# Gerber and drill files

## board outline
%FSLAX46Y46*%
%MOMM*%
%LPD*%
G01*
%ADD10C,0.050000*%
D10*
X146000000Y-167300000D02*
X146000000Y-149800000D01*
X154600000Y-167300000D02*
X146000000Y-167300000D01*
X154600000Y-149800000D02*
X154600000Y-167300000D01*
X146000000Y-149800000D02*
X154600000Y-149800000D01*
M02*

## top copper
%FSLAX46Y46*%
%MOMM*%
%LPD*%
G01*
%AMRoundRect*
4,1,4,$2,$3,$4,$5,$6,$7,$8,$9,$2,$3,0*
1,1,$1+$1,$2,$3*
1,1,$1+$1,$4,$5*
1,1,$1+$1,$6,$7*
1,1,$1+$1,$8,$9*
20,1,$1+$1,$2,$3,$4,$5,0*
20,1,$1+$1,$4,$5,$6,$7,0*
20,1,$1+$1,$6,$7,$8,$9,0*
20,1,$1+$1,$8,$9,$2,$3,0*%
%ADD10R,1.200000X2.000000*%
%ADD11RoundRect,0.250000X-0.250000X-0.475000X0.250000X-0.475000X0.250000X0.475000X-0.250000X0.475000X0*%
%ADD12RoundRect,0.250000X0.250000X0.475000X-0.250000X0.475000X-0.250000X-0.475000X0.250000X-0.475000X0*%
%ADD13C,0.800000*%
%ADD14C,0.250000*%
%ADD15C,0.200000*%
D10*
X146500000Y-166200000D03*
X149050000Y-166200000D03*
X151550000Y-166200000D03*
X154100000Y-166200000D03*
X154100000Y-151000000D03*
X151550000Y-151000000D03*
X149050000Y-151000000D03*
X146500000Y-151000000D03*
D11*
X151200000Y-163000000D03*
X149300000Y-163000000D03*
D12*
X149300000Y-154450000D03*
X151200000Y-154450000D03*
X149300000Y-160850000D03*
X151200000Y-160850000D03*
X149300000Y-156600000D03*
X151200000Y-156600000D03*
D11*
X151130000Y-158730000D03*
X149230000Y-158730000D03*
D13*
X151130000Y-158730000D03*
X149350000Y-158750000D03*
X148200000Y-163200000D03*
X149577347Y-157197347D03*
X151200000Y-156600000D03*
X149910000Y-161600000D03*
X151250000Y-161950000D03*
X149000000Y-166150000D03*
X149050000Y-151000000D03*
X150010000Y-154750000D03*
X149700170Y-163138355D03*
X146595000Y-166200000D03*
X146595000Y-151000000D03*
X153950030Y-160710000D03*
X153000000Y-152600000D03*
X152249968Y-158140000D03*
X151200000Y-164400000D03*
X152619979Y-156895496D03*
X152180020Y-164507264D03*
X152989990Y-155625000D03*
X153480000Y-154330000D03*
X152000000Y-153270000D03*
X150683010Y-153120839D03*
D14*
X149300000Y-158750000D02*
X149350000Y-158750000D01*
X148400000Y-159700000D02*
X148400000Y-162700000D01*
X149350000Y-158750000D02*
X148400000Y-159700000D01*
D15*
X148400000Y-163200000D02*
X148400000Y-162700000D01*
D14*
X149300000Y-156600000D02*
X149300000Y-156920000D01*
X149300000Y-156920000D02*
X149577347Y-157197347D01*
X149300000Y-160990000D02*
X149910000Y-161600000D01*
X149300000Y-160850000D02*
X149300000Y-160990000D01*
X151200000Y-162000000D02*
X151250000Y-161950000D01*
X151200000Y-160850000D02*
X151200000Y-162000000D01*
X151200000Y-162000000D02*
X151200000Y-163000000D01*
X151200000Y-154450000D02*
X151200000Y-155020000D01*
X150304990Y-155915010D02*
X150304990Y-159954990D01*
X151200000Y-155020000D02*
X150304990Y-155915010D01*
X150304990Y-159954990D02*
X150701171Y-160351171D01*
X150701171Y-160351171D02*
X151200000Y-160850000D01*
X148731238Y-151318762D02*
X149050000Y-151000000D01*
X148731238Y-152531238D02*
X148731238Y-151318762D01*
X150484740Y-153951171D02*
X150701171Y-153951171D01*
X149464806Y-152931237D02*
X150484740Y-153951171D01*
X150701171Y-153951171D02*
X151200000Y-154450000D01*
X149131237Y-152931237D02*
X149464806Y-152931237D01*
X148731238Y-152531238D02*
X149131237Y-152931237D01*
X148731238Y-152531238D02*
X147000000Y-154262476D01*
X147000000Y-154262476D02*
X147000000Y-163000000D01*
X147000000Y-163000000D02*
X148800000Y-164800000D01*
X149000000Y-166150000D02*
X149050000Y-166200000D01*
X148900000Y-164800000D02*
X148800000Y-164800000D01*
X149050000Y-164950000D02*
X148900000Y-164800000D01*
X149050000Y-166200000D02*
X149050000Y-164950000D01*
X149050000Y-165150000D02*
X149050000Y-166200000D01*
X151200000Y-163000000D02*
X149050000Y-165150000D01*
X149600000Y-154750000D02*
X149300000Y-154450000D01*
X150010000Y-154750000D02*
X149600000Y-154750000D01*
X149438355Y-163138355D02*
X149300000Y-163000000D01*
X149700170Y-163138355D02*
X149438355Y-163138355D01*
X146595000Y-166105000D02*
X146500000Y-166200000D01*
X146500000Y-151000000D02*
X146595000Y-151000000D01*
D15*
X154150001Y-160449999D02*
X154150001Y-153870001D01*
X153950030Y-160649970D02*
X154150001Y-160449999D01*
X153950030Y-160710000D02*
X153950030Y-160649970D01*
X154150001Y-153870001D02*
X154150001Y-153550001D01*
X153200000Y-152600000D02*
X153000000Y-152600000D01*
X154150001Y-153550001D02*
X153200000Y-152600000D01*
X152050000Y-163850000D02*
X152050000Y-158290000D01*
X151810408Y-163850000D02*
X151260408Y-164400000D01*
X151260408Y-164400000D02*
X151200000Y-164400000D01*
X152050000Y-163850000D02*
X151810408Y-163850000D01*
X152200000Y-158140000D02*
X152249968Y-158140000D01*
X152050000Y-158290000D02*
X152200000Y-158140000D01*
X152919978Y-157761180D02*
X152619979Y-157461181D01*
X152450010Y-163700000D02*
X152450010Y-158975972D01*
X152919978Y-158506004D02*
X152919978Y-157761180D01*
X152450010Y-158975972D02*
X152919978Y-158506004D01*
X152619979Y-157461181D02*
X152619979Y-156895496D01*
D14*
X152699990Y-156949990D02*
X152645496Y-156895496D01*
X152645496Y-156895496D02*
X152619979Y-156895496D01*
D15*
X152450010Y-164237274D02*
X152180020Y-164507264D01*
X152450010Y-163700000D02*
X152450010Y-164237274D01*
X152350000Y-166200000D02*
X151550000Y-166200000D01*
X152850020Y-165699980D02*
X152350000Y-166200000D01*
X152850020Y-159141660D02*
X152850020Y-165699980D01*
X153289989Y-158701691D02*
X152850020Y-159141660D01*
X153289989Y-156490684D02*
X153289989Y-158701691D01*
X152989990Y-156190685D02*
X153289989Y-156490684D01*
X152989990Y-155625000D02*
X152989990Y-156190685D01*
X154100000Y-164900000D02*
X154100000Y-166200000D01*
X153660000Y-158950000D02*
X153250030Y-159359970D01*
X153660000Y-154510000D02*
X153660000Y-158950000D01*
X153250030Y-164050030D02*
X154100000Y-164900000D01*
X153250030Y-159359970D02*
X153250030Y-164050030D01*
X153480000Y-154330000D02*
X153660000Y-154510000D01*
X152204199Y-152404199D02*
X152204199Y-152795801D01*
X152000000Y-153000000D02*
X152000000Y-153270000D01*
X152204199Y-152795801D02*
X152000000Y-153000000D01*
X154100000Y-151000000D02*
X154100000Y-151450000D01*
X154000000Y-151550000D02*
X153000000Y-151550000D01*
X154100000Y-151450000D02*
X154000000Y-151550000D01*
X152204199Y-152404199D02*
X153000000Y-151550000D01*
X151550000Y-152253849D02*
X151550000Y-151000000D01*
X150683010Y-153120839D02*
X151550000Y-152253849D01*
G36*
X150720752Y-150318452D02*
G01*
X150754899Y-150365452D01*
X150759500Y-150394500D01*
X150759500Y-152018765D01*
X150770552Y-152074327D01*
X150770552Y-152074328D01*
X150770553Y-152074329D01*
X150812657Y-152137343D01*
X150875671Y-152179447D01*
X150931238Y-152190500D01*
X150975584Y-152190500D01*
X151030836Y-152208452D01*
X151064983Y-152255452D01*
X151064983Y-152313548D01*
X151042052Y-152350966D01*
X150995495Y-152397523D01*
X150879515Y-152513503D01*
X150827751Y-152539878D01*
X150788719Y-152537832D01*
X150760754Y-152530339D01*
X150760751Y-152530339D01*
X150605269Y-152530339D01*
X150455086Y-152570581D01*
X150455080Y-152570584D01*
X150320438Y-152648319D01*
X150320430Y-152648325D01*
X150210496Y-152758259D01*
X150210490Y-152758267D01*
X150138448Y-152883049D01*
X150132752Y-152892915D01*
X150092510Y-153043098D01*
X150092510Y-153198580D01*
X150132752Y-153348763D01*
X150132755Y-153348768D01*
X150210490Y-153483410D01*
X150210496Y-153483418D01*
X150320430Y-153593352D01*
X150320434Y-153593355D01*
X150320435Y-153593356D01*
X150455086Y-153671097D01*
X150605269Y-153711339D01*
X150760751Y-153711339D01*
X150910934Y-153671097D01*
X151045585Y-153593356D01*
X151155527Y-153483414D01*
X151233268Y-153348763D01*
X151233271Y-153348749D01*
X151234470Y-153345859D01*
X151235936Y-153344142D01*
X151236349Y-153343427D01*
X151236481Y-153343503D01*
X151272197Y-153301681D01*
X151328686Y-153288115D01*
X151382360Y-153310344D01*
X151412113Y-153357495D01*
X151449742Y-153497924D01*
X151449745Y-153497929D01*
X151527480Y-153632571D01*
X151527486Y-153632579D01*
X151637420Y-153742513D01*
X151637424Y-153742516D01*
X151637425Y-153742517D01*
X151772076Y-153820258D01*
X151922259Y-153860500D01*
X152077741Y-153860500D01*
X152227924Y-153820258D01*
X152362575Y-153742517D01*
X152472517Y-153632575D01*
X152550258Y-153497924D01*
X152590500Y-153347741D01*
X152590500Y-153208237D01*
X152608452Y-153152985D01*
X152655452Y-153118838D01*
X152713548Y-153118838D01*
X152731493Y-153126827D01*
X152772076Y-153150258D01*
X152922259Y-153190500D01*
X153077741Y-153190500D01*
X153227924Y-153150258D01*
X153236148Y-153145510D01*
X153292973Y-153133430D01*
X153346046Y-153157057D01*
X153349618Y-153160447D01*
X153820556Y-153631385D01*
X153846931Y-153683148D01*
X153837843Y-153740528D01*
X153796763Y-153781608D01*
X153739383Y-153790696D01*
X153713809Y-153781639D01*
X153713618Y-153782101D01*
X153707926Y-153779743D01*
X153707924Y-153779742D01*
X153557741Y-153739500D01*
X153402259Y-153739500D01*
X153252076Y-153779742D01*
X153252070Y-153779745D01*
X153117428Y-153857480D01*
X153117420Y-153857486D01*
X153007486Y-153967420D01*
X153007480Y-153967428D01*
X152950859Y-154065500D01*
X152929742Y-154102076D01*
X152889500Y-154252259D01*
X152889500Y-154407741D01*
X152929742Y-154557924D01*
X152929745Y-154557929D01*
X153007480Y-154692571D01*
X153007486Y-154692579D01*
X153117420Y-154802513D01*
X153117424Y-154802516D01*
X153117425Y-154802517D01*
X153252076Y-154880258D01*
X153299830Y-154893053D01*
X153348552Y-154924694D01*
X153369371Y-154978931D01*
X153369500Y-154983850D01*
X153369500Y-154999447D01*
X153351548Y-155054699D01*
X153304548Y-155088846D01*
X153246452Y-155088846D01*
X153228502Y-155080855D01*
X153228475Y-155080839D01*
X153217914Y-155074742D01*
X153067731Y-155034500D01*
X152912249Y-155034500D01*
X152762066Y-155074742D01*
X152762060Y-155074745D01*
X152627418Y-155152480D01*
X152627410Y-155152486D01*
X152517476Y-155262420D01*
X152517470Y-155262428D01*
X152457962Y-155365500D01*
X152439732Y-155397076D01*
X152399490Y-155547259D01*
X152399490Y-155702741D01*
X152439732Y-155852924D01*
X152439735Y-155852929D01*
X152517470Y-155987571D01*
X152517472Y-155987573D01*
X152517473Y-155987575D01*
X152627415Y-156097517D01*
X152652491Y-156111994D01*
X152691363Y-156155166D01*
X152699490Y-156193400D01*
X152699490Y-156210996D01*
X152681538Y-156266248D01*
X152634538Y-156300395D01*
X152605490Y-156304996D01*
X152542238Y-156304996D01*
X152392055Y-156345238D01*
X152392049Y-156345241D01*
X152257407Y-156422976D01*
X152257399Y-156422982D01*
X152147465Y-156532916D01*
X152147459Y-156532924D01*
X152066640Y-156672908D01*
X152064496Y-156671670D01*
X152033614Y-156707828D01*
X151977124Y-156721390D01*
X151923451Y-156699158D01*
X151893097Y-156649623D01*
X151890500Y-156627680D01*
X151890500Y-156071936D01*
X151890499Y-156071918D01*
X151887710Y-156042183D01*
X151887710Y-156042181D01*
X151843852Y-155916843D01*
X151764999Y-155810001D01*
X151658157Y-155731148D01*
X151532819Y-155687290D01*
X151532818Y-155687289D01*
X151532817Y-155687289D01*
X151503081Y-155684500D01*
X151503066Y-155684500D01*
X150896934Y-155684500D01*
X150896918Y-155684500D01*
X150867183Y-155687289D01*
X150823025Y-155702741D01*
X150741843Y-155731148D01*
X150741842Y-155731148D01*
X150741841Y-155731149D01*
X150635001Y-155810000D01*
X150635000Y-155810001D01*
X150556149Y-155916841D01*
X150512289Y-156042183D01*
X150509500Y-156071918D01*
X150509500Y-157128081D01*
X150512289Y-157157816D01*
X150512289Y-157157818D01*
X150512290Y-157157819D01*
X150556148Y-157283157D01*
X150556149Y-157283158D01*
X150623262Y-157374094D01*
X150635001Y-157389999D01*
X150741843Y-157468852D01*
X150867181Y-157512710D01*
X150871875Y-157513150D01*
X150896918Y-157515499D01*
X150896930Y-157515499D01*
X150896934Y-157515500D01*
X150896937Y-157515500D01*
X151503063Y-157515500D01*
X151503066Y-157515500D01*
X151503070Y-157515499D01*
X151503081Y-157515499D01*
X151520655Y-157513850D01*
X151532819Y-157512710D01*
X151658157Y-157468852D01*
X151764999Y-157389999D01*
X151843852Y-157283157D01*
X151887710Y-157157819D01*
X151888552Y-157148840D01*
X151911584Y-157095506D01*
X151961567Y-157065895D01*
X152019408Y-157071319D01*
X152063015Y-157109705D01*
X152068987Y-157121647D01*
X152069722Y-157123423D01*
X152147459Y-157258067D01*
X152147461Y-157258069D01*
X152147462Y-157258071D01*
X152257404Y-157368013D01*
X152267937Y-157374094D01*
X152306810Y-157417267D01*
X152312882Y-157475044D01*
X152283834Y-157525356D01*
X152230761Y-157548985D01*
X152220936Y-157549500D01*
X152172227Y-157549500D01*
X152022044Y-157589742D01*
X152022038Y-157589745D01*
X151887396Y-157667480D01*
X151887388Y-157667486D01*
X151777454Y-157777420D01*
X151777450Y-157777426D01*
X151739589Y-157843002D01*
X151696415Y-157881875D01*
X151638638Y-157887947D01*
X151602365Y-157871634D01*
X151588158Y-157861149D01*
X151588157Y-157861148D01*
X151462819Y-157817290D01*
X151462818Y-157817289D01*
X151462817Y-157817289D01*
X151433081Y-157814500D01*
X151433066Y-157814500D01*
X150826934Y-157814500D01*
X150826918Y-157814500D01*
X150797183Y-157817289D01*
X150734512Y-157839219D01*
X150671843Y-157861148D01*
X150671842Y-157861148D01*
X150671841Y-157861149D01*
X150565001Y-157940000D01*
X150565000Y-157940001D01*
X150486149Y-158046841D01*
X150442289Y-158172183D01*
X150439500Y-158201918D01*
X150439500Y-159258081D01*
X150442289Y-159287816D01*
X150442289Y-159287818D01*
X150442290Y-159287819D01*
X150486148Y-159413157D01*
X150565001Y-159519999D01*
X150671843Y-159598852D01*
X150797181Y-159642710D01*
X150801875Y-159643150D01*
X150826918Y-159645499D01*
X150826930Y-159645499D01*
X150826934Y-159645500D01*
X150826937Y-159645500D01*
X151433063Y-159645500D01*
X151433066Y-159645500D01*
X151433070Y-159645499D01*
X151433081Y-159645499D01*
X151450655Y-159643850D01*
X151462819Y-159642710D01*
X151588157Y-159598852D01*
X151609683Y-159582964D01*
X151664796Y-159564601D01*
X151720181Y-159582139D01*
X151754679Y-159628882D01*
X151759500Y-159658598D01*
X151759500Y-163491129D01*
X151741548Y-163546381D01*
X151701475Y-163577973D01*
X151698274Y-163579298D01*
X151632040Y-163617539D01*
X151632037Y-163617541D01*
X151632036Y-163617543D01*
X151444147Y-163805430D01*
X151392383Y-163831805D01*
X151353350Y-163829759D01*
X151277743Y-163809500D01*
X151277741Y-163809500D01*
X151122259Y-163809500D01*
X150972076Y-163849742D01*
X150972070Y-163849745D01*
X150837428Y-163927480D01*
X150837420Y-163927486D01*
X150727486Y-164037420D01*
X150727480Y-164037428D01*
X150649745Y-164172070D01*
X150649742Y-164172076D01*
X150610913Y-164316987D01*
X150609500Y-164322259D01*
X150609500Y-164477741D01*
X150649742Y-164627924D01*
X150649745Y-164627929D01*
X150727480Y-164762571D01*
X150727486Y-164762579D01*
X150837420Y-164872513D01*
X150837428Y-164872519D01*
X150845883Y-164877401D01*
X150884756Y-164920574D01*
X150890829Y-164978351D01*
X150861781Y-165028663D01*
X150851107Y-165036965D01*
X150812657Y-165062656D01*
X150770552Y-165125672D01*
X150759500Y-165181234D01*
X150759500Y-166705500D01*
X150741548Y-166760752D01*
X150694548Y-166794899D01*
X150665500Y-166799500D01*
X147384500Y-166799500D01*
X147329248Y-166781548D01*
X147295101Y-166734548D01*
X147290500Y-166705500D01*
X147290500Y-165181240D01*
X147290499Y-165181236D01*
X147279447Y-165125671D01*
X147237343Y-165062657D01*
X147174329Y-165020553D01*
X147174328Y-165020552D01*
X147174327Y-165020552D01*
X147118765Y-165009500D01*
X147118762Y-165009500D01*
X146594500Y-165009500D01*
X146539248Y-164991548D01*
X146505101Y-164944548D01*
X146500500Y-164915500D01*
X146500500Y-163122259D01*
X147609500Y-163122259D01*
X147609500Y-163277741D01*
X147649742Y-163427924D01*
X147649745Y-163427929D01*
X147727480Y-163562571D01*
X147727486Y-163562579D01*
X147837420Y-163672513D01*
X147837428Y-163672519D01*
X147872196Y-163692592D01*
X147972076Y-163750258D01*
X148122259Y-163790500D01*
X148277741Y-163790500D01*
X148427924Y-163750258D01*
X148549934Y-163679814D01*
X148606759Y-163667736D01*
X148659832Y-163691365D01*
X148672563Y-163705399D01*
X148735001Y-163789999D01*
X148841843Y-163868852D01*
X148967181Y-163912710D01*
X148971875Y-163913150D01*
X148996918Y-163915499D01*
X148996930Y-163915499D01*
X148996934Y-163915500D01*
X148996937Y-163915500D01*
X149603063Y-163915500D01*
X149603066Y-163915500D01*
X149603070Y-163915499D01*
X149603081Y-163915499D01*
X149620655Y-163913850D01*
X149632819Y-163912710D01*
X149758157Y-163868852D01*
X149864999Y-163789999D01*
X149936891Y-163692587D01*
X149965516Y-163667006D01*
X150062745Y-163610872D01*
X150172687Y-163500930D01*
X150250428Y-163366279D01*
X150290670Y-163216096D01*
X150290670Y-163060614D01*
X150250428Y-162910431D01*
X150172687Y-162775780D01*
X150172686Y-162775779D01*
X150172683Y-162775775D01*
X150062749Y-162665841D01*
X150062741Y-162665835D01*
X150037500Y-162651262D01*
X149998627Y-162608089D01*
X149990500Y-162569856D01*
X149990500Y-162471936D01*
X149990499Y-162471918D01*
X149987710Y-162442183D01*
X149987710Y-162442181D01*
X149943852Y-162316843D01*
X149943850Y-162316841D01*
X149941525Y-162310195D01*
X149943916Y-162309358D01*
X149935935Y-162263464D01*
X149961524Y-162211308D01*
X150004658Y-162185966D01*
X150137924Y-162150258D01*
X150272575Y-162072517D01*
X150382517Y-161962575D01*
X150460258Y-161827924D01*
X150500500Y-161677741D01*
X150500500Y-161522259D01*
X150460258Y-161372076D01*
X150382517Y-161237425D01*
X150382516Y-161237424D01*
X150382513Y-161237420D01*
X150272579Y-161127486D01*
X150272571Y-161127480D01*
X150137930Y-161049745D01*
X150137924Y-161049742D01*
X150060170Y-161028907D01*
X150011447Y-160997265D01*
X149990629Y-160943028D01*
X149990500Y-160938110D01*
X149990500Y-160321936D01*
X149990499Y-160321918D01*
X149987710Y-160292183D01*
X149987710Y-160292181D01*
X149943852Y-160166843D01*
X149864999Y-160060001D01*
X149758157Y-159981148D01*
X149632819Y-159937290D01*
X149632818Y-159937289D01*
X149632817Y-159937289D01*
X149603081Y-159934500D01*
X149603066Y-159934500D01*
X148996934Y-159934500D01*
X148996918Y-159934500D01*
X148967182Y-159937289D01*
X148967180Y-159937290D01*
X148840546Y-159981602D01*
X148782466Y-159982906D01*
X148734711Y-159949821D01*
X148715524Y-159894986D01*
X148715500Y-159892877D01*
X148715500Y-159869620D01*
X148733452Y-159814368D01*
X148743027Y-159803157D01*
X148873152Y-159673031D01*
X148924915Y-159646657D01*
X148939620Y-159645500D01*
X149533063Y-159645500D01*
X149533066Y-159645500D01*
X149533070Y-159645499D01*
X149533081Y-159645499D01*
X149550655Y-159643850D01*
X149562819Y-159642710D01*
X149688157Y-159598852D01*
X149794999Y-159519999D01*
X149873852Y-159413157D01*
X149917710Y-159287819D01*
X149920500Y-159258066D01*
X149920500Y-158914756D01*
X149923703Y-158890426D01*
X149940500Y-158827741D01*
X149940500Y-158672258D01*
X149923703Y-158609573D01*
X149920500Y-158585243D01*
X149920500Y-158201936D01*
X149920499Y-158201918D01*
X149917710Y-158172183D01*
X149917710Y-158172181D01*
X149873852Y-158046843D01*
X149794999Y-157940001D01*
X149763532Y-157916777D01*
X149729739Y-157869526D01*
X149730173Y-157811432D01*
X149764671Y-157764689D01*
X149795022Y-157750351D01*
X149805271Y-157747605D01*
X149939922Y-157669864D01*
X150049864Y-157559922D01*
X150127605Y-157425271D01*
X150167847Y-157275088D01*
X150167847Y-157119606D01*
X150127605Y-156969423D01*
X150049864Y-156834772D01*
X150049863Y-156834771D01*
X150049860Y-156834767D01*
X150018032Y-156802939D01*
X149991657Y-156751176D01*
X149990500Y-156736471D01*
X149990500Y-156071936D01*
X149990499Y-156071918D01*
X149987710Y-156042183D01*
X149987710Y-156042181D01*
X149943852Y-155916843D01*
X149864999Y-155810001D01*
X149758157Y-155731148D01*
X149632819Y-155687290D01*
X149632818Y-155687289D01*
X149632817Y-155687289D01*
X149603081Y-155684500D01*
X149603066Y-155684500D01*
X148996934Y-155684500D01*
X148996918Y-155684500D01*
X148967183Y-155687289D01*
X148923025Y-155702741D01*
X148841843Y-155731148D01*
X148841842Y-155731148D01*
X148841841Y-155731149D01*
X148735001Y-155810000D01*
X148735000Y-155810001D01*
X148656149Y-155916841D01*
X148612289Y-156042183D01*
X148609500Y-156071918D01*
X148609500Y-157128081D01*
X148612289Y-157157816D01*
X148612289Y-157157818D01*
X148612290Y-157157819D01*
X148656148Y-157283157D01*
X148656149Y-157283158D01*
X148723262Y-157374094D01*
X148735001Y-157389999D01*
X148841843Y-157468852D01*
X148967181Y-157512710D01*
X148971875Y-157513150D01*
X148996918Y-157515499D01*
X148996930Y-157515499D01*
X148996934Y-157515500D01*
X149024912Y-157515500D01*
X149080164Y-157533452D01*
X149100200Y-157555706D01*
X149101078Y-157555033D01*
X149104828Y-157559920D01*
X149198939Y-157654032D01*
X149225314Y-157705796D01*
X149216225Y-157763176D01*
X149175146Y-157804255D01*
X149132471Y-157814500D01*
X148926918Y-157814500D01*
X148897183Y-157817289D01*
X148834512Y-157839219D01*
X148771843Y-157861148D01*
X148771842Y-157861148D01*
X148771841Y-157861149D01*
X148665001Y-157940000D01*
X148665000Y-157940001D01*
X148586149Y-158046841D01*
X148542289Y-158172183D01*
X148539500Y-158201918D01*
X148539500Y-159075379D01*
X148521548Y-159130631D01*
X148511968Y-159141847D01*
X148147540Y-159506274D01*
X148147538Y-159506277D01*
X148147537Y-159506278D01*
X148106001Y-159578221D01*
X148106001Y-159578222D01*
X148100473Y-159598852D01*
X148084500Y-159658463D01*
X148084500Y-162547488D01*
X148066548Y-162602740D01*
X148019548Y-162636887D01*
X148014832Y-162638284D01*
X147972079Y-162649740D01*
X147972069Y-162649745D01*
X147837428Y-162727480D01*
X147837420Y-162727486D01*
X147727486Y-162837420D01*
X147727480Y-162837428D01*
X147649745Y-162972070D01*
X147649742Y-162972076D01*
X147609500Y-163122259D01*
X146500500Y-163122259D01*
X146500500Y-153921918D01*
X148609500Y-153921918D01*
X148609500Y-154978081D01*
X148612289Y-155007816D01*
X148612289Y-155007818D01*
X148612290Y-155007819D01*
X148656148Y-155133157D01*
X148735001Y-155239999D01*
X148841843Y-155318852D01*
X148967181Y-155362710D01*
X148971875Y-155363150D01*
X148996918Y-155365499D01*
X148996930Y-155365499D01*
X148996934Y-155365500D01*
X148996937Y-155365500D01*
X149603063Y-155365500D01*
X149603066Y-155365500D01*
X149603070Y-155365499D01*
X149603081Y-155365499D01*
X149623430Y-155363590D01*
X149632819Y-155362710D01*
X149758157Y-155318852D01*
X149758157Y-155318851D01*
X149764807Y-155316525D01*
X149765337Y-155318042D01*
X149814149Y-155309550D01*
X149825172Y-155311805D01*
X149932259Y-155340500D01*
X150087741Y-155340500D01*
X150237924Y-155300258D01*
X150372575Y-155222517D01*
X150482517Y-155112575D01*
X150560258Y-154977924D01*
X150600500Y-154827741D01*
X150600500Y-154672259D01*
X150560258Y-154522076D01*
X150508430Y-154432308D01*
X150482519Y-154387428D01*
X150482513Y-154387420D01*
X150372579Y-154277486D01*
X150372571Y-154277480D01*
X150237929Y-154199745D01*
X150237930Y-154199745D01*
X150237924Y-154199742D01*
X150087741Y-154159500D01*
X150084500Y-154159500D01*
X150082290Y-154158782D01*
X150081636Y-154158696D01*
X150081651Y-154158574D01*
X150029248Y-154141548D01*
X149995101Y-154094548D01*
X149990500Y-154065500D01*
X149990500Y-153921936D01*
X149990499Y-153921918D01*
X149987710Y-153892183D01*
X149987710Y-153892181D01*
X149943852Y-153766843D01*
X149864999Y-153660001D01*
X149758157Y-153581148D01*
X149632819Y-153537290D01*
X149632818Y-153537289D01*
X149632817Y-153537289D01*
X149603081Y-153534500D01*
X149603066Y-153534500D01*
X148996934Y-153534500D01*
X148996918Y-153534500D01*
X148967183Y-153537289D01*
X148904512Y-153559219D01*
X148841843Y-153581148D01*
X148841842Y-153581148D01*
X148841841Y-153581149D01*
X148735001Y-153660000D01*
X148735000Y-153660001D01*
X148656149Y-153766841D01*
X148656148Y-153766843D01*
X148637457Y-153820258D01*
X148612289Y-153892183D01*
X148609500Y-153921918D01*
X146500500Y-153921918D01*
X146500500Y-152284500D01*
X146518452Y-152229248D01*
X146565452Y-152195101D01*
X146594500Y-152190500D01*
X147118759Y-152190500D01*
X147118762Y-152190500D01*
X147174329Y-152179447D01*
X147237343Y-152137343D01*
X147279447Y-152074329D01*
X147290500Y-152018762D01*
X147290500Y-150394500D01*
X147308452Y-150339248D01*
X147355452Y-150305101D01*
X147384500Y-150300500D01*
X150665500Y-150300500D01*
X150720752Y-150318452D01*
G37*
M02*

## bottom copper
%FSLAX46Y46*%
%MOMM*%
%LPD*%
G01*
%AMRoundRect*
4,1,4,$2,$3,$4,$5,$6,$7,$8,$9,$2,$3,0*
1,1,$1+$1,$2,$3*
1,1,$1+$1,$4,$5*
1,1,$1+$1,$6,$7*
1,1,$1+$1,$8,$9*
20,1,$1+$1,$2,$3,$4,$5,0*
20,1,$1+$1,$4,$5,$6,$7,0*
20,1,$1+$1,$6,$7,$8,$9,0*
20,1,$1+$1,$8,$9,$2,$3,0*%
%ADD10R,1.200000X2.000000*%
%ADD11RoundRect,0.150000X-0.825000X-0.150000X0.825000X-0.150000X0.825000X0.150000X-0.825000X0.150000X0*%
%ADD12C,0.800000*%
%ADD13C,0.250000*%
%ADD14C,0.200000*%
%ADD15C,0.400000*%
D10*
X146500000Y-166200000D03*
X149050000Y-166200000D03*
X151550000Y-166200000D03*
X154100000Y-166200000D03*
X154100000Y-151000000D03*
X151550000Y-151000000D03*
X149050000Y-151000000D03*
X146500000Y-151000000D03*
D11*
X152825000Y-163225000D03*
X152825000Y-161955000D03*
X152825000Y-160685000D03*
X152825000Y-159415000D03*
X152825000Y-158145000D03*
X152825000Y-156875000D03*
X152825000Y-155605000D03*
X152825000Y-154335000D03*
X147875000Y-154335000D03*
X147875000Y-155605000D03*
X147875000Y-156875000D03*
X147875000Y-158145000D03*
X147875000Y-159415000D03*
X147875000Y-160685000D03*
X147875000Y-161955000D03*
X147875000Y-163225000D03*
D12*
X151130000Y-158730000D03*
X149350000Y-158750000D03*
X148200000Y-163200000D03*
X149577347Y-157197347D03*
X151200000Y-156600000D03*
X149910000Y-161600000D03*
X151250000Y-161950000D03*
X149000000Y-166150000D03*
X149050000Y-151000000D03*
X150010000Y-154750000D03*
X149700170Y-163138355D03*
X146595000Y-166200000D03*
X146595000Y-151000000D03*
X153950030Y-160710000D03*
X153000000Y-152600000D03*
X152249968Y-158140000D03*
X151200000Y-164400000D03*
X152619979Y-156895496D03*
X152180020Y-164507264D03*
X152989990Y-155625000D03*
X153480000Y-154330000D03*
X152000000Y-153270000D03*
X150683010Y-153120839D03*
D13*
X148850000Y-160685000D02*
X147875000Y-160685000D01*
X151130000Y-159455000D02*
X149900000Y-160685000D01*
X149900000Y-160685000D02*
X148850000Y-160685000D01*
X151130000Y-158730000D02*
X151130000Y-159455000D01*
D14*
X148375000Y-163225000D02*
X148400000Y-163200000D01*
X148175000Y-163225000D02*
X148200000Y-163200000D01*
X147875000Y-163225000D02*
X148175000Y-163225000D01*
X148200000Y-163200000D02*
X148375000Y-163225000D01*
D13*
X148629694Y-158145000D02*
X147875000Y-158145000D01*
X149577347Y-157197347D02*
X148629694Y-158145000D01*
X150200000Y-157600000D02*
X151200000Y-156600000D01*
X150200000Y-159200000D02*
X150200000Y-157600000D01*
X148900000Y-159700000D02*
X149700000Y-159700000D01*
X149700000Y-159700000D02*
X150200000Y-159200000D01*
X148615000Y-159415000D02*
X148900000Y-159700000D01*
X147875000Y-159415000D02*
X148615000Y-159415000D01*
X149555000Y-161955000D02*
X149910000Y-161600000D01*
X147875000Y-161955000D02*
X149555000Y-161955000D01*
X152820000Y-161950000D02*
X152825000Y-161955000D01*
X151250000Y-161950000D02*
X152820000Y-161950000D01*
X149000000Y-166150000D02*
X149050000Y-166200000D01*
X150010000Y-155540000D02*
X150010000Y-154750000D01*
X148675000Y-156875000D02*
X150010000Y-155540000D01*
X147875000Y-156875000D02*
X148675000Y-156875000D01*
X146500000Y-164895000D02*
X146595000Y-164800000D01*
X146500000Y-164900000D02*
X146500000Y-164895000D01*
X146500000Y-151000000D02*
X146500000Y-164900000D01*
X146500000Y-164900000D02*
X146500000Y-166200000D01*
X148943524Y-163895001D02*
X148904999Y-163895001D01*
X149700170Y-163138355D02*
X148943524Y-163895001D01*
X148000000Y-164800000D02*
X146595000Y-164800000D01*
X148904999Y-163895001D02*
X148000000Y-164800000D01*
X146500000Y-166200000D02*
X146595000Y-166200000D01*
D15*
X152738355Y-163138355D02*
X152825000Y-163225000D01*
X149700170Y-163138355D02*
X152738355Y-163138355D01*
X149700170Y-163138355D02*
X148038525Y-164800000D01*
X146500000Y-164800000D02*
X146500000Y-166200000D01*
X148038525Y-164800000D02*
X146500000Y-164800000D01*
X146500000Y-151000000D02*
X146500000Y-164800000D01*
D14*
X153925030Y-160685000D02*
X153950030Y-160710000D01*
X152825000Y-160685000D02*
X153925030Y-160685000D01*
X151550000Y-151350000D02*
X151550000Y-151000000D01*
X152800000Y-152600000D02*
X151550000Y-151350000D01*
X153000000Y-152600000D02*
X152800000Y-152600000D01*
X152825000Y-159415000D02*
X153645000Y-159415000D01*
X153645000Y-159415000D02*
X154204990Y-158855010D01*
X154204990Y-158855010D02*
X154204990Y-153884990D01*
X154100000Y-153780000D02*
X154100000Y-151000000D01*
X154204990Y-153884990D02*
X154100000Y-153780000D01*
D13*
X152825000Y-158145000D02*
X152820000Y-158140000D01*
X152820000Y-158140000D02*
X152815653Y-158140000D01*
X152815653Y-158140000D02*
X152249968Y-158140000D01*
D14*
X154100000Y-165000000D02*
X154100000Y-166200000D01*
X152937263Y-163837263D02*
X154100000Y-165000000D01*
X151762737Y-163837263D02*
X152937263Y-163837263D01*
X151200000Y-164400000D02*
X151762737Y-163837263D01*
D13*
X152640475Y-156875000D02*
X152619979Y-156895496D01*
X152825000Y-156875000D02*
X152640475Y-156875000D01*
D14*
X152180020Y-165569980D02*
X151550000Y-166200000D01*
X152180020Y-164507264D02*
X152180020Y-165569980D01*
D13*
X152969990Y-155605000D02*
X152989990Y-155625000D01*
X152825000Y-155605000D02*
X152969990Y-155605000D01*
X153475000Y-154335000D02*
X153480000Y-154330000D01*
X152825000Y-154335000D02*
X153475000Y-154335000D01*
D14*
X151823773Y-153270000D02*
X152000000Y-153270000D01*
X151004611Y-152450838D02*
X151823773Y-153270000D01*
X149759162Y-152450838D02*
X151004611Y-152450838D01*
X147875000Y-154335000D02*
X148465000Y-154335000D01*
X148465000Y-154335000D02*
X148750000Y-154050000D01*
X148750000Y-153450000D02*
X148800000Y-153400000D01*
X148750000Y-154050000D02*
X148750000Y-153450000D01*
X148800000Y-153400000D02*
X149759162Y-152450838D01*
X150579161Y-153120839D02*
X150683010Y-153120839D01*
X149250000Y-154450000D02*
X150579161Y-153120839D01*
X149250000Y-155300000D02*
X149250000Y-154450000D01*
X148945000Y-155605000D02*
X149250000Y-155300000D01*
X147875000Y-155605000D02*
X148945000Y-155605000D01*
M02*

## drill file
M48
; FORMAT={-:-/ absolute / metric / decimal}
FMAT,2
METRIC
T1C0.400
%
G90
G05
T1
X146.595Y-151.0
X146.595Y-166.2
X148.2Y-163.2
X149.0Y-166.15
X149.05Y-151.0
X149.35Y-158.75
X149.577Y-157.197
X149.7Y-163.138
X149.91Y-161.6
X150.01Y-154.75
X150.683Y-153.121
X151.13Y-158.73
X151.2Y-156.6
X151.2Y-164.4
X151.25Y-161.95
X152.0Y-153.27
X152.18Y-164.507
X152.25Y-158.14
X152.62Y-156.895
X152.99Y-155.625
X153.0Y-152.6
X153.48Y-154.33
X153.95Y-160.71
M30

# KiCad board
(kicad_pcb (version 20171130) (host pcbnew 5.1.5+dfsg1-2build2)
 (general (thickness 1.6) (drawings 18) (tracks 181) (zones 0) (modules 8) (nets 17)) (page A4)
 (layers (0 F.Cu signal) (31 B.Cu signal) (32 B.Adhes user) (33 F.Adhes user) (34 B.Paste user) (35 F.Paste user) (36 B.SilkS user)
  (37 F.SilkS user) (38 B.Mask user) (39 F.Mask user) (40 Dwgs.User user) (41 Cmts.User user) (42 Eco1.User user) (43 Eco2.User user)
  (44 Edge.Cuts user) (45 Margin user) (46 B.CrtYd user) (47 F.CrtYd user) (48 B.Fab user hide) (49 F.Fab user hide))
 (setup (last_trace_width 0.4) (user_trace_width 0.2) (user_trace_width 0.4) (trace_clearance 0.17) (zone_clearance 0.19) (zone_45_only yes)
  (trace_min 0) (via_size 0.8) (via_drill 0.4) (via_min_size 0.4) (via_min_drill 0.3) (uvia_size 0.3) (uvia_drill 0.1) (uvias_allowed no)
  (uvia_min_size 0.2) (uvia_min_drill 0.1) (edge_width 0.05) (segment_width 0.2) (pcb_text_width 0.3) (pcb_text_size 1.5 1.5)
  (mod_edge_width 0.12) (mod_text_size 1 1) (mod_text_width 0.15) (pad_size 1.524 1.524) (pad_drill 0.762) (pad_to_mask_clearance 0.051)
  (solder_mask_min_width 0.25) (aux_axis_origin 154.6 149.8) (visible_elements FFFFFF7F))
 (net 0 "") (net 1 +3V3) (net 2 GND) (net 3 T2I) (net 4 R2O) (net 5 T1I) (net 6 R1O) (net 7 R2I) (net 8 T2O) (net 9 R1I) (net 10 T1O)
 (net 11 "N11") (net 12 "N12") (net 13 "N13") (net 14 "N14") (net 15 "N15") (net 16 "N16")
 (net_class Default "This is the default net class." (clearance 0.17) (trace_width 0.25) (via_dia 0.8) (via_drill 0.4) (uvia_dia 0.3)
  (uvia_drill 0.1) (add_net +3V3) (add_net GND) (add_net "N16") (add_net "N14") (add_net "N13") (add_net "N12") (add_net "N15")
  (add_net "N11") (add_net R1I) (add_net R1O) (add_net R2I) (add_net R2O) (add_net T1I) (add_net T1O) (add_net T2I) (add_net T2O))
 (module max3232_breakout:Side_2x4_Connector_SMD (layer B.Cu) (at 150.3 166.2 270)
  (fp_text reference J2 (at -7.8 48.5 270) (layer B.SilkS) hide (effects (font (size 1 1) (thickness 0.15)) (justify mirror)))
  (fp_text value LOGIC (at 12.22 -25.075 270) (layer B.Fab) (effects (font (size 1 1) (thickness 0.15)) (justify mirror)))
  (pad 8 smd rect (at 0 3.8 270) (size 2 1.2) (layers F.Cu F.Paste F.Mask) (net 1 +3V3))
  (pad 6 smd rect (at 0 1.25 270) (size 2 1.2) (layers F.Cu F.Paste F.Mask) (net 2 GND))
  (pad 4 smd rect (at 0 -1.25 270) (size 2 1.2) (layers F.Cu F.Paste F.Mask) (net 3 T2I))
  (pad 2 smd rect (at 0 -3.8 270) (size 2 1.2) (layers F.Cu F.Paste F.Mask) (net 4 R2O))
  (pad 7 smd rect (at 0 3.8 270) (size 2 1.2) (layers B.Cu B.Paste B.Mask) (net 1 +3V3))
  (pad 5 smd rect (at 0 1.25 270) (size 2 1.2) (layers B.Cu B.Paste B.Mask) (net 2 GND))
  (pad 3 smd rect (at 0 -1.25 270) (size 2 1.2) (layers B.Cu B.Paste B.Mask) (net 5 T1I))
  (pad 1 smd rect (at 0 -3.8 270) (size 2 1.2) (layers B.Cu B.Paste B.Mask) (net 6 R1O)))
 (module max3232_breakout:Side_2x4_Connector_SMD (layer B.Cu) (at 150.3 151 90)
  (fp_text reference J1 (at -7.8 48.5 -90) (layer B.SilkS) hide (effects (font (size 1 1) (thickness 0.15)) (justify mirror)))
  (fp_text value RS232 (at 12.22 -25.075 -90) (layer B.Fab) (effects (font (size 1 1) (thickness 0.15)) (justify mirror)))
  (pad 8 smd rect (at 0 3.8 90) (size 2 1.2) (layers F.Cu F.Paste F.Mask) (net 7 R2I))
  (pad 6 smd rect (at 0 1.25 90) (size 2 1.2) (layers F.Cu F.Paste F.Mask) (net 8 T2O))
  (pad 4 smd rect (at 0 -1.25 90) (size 2 1.2) (layers F.Cu F.Paste F.Mask) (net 2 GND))
  (pad 2 smd rect (at 0 -3.8 90) (size 2 1.2) (layers F.Cu F.Paste F.Mask) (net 1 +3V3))
  (pad 7 smd rect (at 0 3.8 90) (size 2 1.2) (layers B.Cu B.Paste B.Mask) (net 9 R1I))
  (pad 5 smd rect (at 0 1.25 90) (size 2 1.2) (layers B.Cu B.Paste B.Mask) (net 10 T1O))
  (pad 3 smd rect (at 0 -1.25 90) (size 2 1.2) (layers B.Cu B.Paste B.Mask) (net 2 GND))
  (pad 1 smd rect (at 0 -3.8 90) (size 2 1.2) (layers B.Cu B.Paste B.Mask) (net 1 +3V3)))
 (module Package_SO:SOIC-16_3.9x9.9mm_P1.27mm (layer B.Cu) (at 150.35 158.78)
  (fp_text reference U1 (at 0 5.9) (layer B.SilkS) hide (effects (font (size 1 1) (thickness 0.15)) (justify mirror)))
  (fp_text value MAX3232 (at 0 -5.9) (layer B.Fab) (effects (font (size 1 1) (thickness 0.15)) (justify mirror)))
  (pad 16 smd roundrect (at 2.475 4.445) (size 1.95 0.6) (layers B.Cu B.Paste B.Mask) (roundrect_rratio 0.25) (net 1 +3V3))
  (pad 15 smd roundrect (at 2.475 3.175) (size 1.95 0.6) (layers B.Cu B.Paste B.Mask) (roundrect_rratio 0.25) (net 2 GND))
  (pad 14 smd roundrect (at 2.475 1.905) (size 1.95 0.6) (layers B.Cu B.Paste B.Mask) (roundrect_rratio 0.25) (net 10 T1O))
  (pad 13 smd roundrect (at 2.475 0.635) (size 1.95 0.6) (layers B.Cu B.Paste B.Mask) (roundrect_rratio 0.25) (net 9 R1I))
  (pad 12 smd roundrect (at 2.475 -0.635) (size 1.95 0.6) (layers B.Cu B.Paste B.Mask) (roundrect_rratio 0.25) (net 6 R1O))
  (pad 11 smd roundrect (at 2.475 -1.905) (size 1.95 0.6) (layers B.Cu B.Paste B.Mask) (roundrect_rratio 0.25) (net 5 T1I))
  (pad 10 smd roundrect (at 2.475 -3.175) (size 1.95 0.6) (layers B.Cu B.Paste B.Mask) (roundrect_rratio 0.25) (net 3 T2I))
  (pad 9 smd roundrect (at 2.475 -4.445) (size 1.95 0.6) (layers B.Cu B.Paste B.Mask) (roundrect_rratio 0.25) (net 4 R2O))
  (pad 8 smd roundrect (at -2.475 -4.445) (size 1.95 0.6) (layers B.Cu B.Paste B.Mask) (roundrect_rratio 0.25) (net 7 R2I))
  (pad 7 smd roundrect (at -2.475 -3.175) (size 1.95 0.6) (layers B.Cu B.Paste B.Mask) (roundrect_rratio 0.25) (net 8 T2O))
  (pad 6 smd roundrect (at -2.475 -1.905) (size 1.95 0.6) (layers B.Cu B.Paste B.Mask) (roundrect_rratio 0.25) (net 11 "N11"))
  (pad 5 smd roundrect (at -2.475 -0.635) (size 1.95 0.6) (layers B.Cu B.Paste B.Mask) (roundrect_rratio 0.25) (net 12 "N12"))
  (pad 4 smd roundrect (at -2.475 0.635) (size 1.95 0.6) (layers B.Cu B.Paste B.Mask) (roundrect_rratio 0.25) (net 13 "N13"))
  (pad 3 smd roundrect (at -2.475 1.905) (size 1.95 0.6) (layers B.Cu B.Paste B.Mask) (roundrect_rratio 0.25) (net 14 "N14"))
  (pad 2 smd roundrect (at -2.475 3.175) (size 1.95 0.6) (layers B.Cu B.Paste B.Mask) (roundrect_rratio 0.25) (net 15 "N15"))
  (pad 1 smd roundrect (at -2.475 4.445) (size 1.95 0.6) (layers B.Cu B.Paste B.Mask) (roundrect_rratio 0.25) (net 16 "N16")))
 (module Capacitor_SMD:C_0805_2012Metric (layer F.Cu) (at 150.25 163)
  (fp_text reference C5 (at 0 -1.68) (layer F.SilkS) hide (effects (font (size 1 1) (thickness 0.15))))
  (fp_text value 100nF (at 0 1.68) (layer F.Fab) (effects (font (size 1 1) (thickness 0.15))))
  (pad 2 smd roundrect (at 0.95 0) (size 1 1.45) (layers F.Cu F.Paste F.Mask) (roundrect_rratio 0.25) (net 2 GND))
  (pad 1 smd roundrect (at -0.95 0) (size 1 1.45) (layers F.Cu F.Paste F.Mask) (roundrect_rratio 0.25) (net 1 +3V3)))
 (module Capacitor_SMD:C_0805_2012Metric (layer F.Cu) (at 150.25 154.45 180)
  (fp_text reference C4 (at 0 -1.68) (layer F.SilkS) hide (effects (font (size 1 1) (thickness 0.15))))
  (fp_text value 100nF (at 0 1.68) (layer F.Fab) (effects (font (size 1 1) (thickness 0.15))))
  (pad 2 smd roundrect (at 0.95 0 180) (size 1 1.45) (layers F.Cu F.Paste F.Mask) (roundrect_rratio 0.25) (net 11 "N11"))
  (pad 1 smd roundrect (at -0.95 0 180) (size 1 1.45) (layers F.Cu F.Paste F.Mask) (roundrect_rratio 0.25) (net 2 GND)))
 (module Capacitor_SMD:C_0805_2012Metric (layer F.Cu) (at 150.25 160.85 180)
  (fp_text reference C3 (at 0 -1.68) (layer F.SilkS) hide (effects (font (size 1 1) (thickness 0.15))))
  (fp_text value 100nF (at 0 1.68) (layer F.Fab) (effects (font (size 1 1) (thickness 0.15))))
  (pad 2 smd roundrect (at 0.95 0 180) (size 1 1.45) (layers F.Cu F.Paste F.Mask) (roundrect_rratio 0.25) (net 15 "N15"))
  (pad 1 smd roundrect (at -0.95 0 180) (size 1 1.45) (layers F.Cu F.Paste F.Mask) (roundrect_rratio 0.25) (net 2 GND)))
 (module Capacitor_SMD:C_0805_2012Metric (layer F.Cu) (at 150.25 156.6 180)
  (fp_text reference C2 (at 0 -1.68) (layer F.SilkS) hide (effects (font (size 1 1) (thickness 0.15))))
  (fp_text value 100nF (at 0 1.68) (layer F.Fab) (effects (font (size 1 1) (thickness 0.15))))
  (pad 2 smd roundrect (at 0.95 0 180) (size 1 1.45) (layers F.Cu F.Paste F.Mask) (roundrect_rratio 0.25) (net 12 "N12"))
  (pad 1 smd roundrect (at -0.95 0 180) (size 1 1.45) (layers F.Cu F.Paste F.Mask) (roundrect_rratio 0.25) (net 13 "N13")))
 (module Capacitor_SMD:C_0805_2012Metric (layer F.Cu) (at 150.18 158.73)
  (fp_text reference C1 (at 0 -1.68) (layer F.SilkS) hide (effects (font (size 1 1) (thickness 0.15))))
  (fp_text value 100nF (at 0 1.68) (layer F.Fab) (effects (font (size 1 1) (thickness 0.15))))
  (pad 2 smd roundrect (at 0.95 0) (size 1 1.45) (layers F.Cu F.Paste F.Mask) (roundrect_rratio 0.25) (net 14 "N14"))
  (pad 1 smd roundrect (at -0.95 0) (size 1 1.45) (layers F.Cu F.Paste F.Mask) (roundrect_rratio 0.25) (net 16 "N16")))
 (gr_line (start 146 167.3) (end 146 149.8) (layer Edge.Cuts) (width 0.05))
 (gr_line (start 154.6 167.3) (end 146 167.3) (layer Edge.Cuts) (width 0.05))
 (gr_line (start 154.6 149.8) (end 154.6 167.3) (layer Edge.Cuts) (width 0.05))
 (gr_line (start 146 149.8) (end 154.6 149.8) (layer Edge.Cuts) (width 0.05))
 (via (at 151.13 158.73) (size 0.8) (drill 0.4) (layers F.Cu B.Cu) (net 14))
 (segment (start 148.85 160.685) (end 147.875 160.685) (width 0.25) (layer B.Cu) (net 14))
 (segment (start 151.13 159.455) (end 149.9 160.685) (width 0.25) (layer B.Cu) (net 14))
 (segment (start 149.9 160.685) (end 148.85 160.685) (width 0.25) (layer B.Cu) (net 14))
 (segment (start 151.13 158.73) (end 151.13 159.455) (width 0.25) (layer B.Cu) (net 14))
 (via (at 149.35 158.75) (size 0.8) (drill 0.4) (layers F.Cu B.Cu) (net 16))
 (segment (start 149.3 158.75) (end 149.35 158.75) (width 0.25) (layer F.Cu) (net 16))
 (segment (start 148.4 159.7) (end 148.4 162.7) (width 0.25) (layer F.Cu) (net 16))
 (segment (start 149.35 158.75) (end 148.4 159.7) (width 0.25) (layer F.Cu) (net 16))
 (segment (start 148.375 163.225) (end 148.4 163.2) (width 0.2) (layer B.Cu) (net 16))
 (segment (start 148.4 163.2) (end 148.4 162.7) (width 0.2) (layer F.Cu) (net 16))
 (via (at 148.2 163.2) (size 0.8) (drill 0.4) (layers F.Cu B.Cu) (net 16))
 (segment (start 148.175 163.225) (end 148.2 163.2) (width 0.2) (layer B.Cu) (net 16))
 (segment (start 147.875 163.225) (end 148.175 163.225) (width 0.2) (layer B.Cu) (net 16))
 (segment (start 148.2 163.2) (end 148.375 163.225) (width 0.2) (layer B.Cu) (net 16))
 (segment (start 148.629694 158.145) (end 147.875 158.145) (width 0.25) (layer B.Cu) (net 12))
 (segment (start 149.3 156.6) (end 149.3 156.92) (width 0.25) (layer F.Cu) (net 12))
 (via (at 149.577347 157.197347) (size 0.8) (drill 0.4) (layers F.Cu B.Cu) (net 12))
 (segment (start 149.3 156.92) (end 149.577347 157.197347) (width 0.25) (layer F.Cu) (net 12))
 (segment (start 149.577347 157.197347) (end 148.629694 158.145) (width 0.25) (layer B.Cu) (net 12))
 (via (at 151.2 156.6) (size 0.8) (drill 0.4) (layers F.Cu B.Cu) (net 13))
 (segment (start 150.2 157.6) (end 151.2 156.6) (width 0.25) (layer B.Cu) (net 13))
 (segment (start 150.2 159.2) (end 150.2 157.6) (width 0.25) (layer B.Cu) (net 13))
 (segment (start 148.9 159.7) (end 149.7 159.7) (width 0.25) (layer B.Cu) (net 13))
 (segment (start 149.7 159.7) (end 150.2 159.2) (width 0.25) (layer B.Cu) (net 13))
 (segment (start 148.615 159.415) (end 148.9 159.7) (width 0.25) (layer B.Cu) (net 13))
 (segment (start 147.875 159.415) (end 148.615 159.415) (width 0.25) (layer B.Cu) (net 13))
 (via (at 149.91 161.6) (size 0.8) (drill 0.4) (layers F.Cu B.Cu) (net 15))
 (segment (start 149.3 160.99) (end 149.91 161.6) (width 0.25) (layer F.Cu) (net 15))
 (segment (start 149.3 160.85) (end 149.3 160.99) (width 0.25) (layer F.Cu) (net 15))
 (segment (start 149.555 161.955) (end 149.91 161.6) (width 0.25) (layer B.Cu) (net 15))
 (segment (start 147.875 161.955) (end 149.555 161.955) (width 0.25) (layer B.Cu) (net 15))
 (segment (start 151.2 162) (end 151.25 161.95) (width 0.25) (layer F.Cu) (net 2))
 (via (at 151.25 161.95) (size 0.8) (drill 0.4) (layers F.Cu B.Cu) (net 2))
 (segment (start 151.2 160.85) (end 151.2 162) (width 0.25) (layer F.Cu) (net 2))
 (segment (start 151.2 162) (end 151.2 163) (width 0.25) (layer F.Cu) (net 2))
 (segment (start 152.82 161.95) (end 152.825 161.955) (width 0.25) (layer B.Cu) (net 2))
 (segment (start 151.25 161.95) (end 152.82 161.95) (width 0.25) (layer B.Cu) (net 2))
 (segment (start 151.2 154.45) (end 151.2 155.02) (width 0.25) (layer F.Cu) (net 2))
 (segment (start 150.30499 155.91501) (end 150.30499 159.95499) (width 0.25) (layer F.Cu) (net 2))
 (segment (start 151.2 155.02) (end 150.30499 155.91501) (width 0.25) (layer F.Cu) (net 2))
 (segment (start 150.30499 159.95499) (end 150.701171 160.351171) (width 0.25) (layer F.Cu) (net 2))
 (segment (start 150.701171 160.351171) (end 151.2 160.85) (width 0.25) (layer F.Cu) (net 2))
 (segment (start 148.731238 151.318762) (end 149.05 151) (width 0.25) (layer F.Cu) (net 2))
 (segment (start 148.731238 152.531238) (end 148.731238 151.318762) (width 0.25) (layer F.Cu) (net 2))
 (segment (start 150.48474 153.951171) (end 150.701171 153.951171) (width 0.25) (layer F.Cu) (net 2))
 (segment (start 149.464806 152.931237) (end 150.48474 153.951171) (width 0.25) (layer F.Cu) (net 2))
 (segment (start 150.701171 153.951171) (end 151.2 154.45) (width 0.25) (layer F.Cu) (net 2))
 (segment (start 149.131237 152.931237) (end 149.464806 152.931237) (width 0.25) (layer F.Cu) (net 2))
 (segment (start 148.731238 152.531238) (end 149.131237 152.931237) (width 0.25) (layer F.Cu) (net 2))
 (segment (start 148.731238 152.531238) (end 147 154.262476) (width 0.25) (layer F.Cu) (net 2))
 (segment (start 147 154.262476) (end 147 163) (width 0.25) (layer F.Cu) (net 2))
 (segment (start 147 163) (end 148.8 164.8) (width 0.25) (layer F.Cu) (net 2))
 (segment (start 149 166.15) (end 149.05 166.2) (width 0.25) (layer B.Cu) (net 2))
 (segment (start 149 166.15) (end 149.05 166.2) (width 0.25) (layer F.Cu) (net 2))
 (segment (start 148.9 164.8) (end 148.8 164.8) (width 0.25) (layer F.Cu) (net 2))
 (segment (start 149.05 164.95) (end 148.9 164.8) (width 0.25) (layer F.Cu) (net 2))
 (segment (start 149.05 166.2) (end 149.05 164.95) (width 0.25) (layer F.Cu) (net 2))
 (via (at 149 166.15) (size 0.8) (drill 0.4) (layers F.Cu B.Cu) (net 2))
 (via (at 149.05 151) (size 0.8) (drill 0.4) (layers F.Cu B.Cu) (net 2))
 (segment (start 149.05 165.15) (end 149.05 166.2) (width 0.25) (layer F.Cu) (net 2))
 (segment (start 151.2 163) (end 149.05 165.15) (width 0.25) (layer F.Cu) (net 2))
 (via (at 150.01 154.75) (size 0.8) (drill 0.4) (layers F.Cu B.Cu) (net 11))
 (segment (start 149.6 154.75) (end 149.3 154.45) (width 0.25) (layer F.Cu) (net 11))
 (segment (start 150.01 154.75) (end 149.6 154.75) (width 0.25) (layer F.Cu) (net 11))
 (segment (start 150.01 155.54) (end 150.01 154.75) (width 0.25) (layer B.Cu) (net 11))
 (segment (start 148.675 156.875) (end 150.01 155.54) (width 0.25) (layer B.Cu) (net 11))
 (segment (start 147.875 156.875) (end 148.675 156.875) (width 0.25) (layer B.Cu) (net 11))
 (via (at 149.70017 163.138355) (size 0.8) (drill 0.4) (layers F.Cu B.Cu) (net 1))
 (segment (start 149.438355 163.138355) (end 149.3 163) (width 0.25) (layer F.Cu) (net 1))
 (segment (start 149.70017 163.138355) (end 149.438355 163.138355) (width 0.25) (layer F.Cu) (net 1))
 (segment (start 146.5 164.895) (end 146.595 164.8) (width 0.25) (layer B.Cu) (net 1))
 (segment (start 146.5 164.9) (end 146.5 164.895) (width 0.25) (layer B.Cu) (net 1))
 (segment (start 146.5 151) (end 146.5 164.9) (width 0.25) (layer B.Cu) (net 1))
 (segment (start 146.5 164.9) (end 146.5 166.2) (width 0.25) (layer B.Cu) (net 1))
 (segment (start 146.595 166.105) (end 146.5 166.2) (width 0.25) (layer F.Cu) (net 1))
 (segment (start 148.943524 163.895001) (end 148.904999 163.895001) (width 0.25) (layer B.Cu) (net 1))
 (segment (start 149.70017 163.138355) (end 148.943524 163.895001) (width 0.25) (layer B.Cu) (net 1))
 (segment (start 148 164.8) (end 146.595 164.8) (width 0.25) (layer B.Cu) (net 1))
 (segment (start 148.904999 163.895001) (end 148 164.8) (width 0.25) (layer B.Cu) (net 1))
 (via (at 146.595 166.2) (size 0.8) (drill 0.4) (layers F.Cu B.Cu) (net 1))
 (segment (start 146.5 166.2) (end 146.595 166.2) (width 0.25) (layer B.Cu) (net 1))
 (via (at 146.595 151) (size 0.8) (drill 0.4) (layers F.Cu B.Cu) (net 1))
 (segment (start 146.5 151) (end 146.595 151) (width 0.25) (layer F.Cu) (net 1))
 (segment (start 152.738355 163.138355) (end 152.825 163.225) (width 0.4) (layer B.Cu) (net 1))
 (segment (start 149.70017 163.138355) (end 152.738355 163.138355) (width 0.4) (layer B.Cu) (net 1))
 (segment (start 149.70017 163.138355) (end 148.038525 164.8) (width 0.4) (layer B.Cu) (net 1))
 (segment (start 146.5 164.8) (end 146.5 166.2) (width 0.4) (layer B.Cu) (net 1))
 (segment (start 148.038525 164.8) (end 146.5 164.8) (width 0.4) (layer B.Cu) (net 1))
 (segment (start 146.5 151) (end 146.5 164.8) (width 0.4) (layer B.Cu) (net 1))
 (via (at 153.95003 160.71) (size 0.8) (drill 0.4) (layers F.Cu B.Cu) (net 10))
 (segment (start 153.92503 160.685) (end 153.95003 160.71) (width 0.2) (layer B.Cu) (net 10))
 (segment (start 152.825 160.685) (end 153.92503 160.685) (width 0.2) (layer B.Cu) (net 10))
 (segment (start 154.150001 160.449999) (end 154.150001 153.870001) (width 0.2) (layer F.Cu) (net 10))
 (segment (start 153.95003 160.64997) (end 154.150001 160.449999) (width 0.2) (layer F.Cu) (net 10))
 (segment (start 153.95003 160.71) (end 153.95003 160.64997) (width 0.2) (layer F.Cu) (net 10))
 (segment (start 154.150001 153.870001) (end 154.150001 153.550001) (width 0.2) (layer F.Cu) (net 10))
 (segment (start 153.2 152.6) (end 153 152.6) (width 0.2) (layer F.Cu) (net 10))
 (via (at 153 152.6) (size 0.8) (drill 0.4) (layers F.Cu B.Cu) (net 10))
 (segment (start 154.150001 153.550001) (end 153.2 152.6) (width 0.2) (layer F.Cu) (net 10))
 (segment (start 151.55 151.35) (end 151.55 151) (width 0.2) (layer B.Cu) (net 10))
 (segment (start 152.8 152.6) (end 151.55 151.35) (width 0.2) (layer B.Cu) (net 10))
 (segment (start 153 152.6) (end 152.8 152.6) (width 0.2) (layer B.Cu) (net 10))
 (segment (start 152.825 159.415) (end 153.645 159.415) (width 0.2) (layer B.Cu) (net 9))
 (segment (start 153.645 159.415) (end 154.20499 158.85501) (width 0.2) (layer B.Cu) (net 9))
 (segment (start 154.20499 158.85501) (end 154.20499 153.88499) (width 0.2) (layer B.Cu) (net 9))
 (segment (start 154.1 153.78) (end 154.1 151) (width 0.2) (layer B.Cu) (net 9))
 (segment (start 154.20499 153.88499) (end 154.1 153.78) (width 0.2) (layer B.Cu) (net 9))
 (via (at 152.249968 158.14) (size 0.8) (drill 0.4) (layers F.Cu B.Cu) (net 6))
 (segment (start 152.825 158.145) (end 152.82 158.14) (width 0.25) (layer B.Cu) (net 6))
 (segment (start 152.82 158.14) (end 152.815653 158.14) (width 0.25) (layer B.Cu) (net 6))
 (segment (start 152.815653 158.14) (end 152.249968 158.14) (width 0.25) (layer B.Cu) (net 6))
 (via (at 151.2 164.4) (size 0.8) (drill 0.4) (layers F.Cu B.Cu) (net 6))
 (segment (start 154.1 165) (end 154.1 166.2) (width 0.2) (layer B.Cu) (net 6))
 (segment (start 152.937263 163.837263) (end 154.1 165) (width 0.2) (layer B.Cu) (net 6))
 (segment (start 151.762737 163.837263) (end 152.937263 163.837263) (width 0.2) (layer B.Cu) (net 6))
 (segment (start 151.2 164.4) (end 151.762737 163.837263) (width 0.2) (layer B.Cu) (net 6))
 (segment (start 152.05 163.85) (end 152.05 158.29) (width 0.2) (layer F.Cu) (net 6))
 (segment (start 151.810408 163.85) (end 151.260408 164.4) (width 0.2) (layer F.Cu) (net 6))
 (segment (start 151.260408 164.4) (end 151.2 164.4) (width 0.2) (layer F.Cu) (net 6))
 (segment (start 152.05 163.85) (end 151.810408 163.85) (width 0.2) (layer F.Cu) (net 6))
 (segment (start 152.2 158.14) (end 152.249968 158.14) (width 0.2) (layer F.Cu) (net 6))
 (segment (start 152.05 158.29) (end 152.2 158.14) (width 0.2) (layer F.Cu) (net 6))
 (segment (start 152.919978 157.76118) (end 152.619979 157.461181) (width 0.2) (layer F.Cu) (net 5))
 (segment (start 152.45001 163.7) (end 152.45001 158.975972) (width 0.2) (layer F.Cu) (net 5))
 (segment (start 152.919978 158.506004) (end 152.919978 157.76118) (width 0.2) (layer F.Cu) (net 5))
 (via (at 152.619979 156.895496) (size 0.8) (drill 0.4) (layers F.Cu B.Cu) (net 5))
 (segment (start 152.45001 158.975972) (end 152.919978 158.506004) (width 0.2) (layer F.Cu) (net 5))
 (segment (start 152.619979 157.461181) (end 152.619979 156.895496) (width 0.2) (layer F.Cu) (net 5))
 (segment (start 152.69999 156.94999) (end 152.645496 156.895496) (width 0.25) (layer F.Cu) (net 5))
 (segment (start 152.640475 156.875) (end 152.619979 156.895496) (width 0.25) (layer B.Cu) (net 5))
 (segment (start 152.825 156.875) (end 152.640475 156.875) (width 0.25) (layer B.Cu) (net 5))
 (segment (start 152.645496 156.895496) (end 152.619979 156.895496) (width 0.25) (layer F.Cu) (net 5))
 (via (at 152.18002 164.507264) (size 0.8) (drill 0.4) (layers F.Cu B.Cu) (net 5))
 (segment (start 152.45001 164.237274) (end 152.18002 164.507264) (width 0.2) (layer F.Cu) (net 5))
 (segment (start 152.45001 163.7) (end 152.45001 164.237274) (width 0.2) (layer F.Cu) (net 5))
 (segment (start 152.18002 165.56998) (end 151.55 166.2) (width 0.2) (layer B.Cu) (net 5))
 (segment (start 152.18002 164.507264) (end 152.18002 165.56998) (width 0.2) (layer B.Cu) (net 5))
 (via (at 152.98999 155.625) (size 0.8) (drill 0.4) (layers F.Cu B.Cu) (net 3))
 (segment (start 152.96999 155.605) (end 152.98999 155.625) (width 0.25) (layer B.Cu) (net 3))
 (segment (start 152.825 155.605) (end 152.96999 155.605) (width 0.25) (layer B.Cu) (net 3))
 (segment (start 152.35 166.2) (end 151.55 166.2) (width 0.2) (layer F.Cu) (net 3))
 (segment (start 152.85002 165.69998) (end 152.35 166.2) (width 0.2) (layer F.Cu) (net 3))
 (segment (start 152.85002 159.14166) (end 152.85002 165.69998) (width 0.2) (layer F.Cu) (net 3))
 (segment (start 153.289989 158.701691) (end 152.85002 159.14166) (width 0.2) (layer F.Cu) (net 3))
 (segment (start 153.289989 156.490684) (end 153.289989 158.701691) (width 0.2) (layer F.Cu) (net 3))
 (segment (start 152.98999 156.190685) (end 153.289989 156.490684) (width 0.2) (layer F.Cu) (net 3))
 (segment (start 152.98999 155.625) (end 152.98999 156.190685) (width 0.2) (layer F.Cu) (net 3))
 (segment (start 153.475 154.335) (end 153.48 154.33) (width 0.25) (layer B.Cu) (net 4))
 (via (at 153.48 154.33) (size 0.8) (drill 0.4) (layers F.Cu B.Cu) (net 4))
 (segment (start 152.825 154.335) (end 153.475 154.335) (width 0.25) (layer B.Cu) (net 4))
 (segment (start 154.1 164.9) (end 154.1 166.2) (width 0.2) (layer F.Cu) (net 4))
 (segment (start 153.66 158.95) (end 153.25003 159.35997) (width 0.2) (layer F.Cu) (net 4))
 (segment (start 153.66 154.51) (end 153.66 158.95) (width 0.2) (layer F.Cu) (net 4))
 (segment (start 153.25003 164.05003) (end 154.1 164.9) (width 0.2) (layer F.Cu) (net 4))
 (segment (start 153.25003 159.35997) (end 153.25003 164.05003) (width 0.2) (layer F.Cu) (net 4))
 (segment (start 153.48 154.33) (end 153.66 154.51) (width 0.2) (layer F.Cu) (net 4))
 (segment (start 151.823773 153.27) (end 152 153.27) (width 0.2) (layer B.Cu) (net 7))
 (via (at 152 153.27) (size 0.8) (drill 0.4) (layers F.Cu B.Cu) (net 7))
 (segment (start 151.004611 152.450838) (end 151.823773 153.27) (width 0.2) (layer B.Cu) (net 7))
 (segment (start 149.759162 152.450838) (end 151.004611 152.450838) (width 0.2) (layer B.Cu) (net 7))
 (segment (start 152.204199 152.404199) (end 152.204199 152.795801) (width 0.2) (layer F.Cu) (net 7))
 (segment (start 152 153) (end 152 153.27) (width 0.2) (layer F.Cu) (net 7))
 (segment (start 152.204199 152.795801) (end 152 153) (width 0.2) (layer F.Cu) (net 7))
 (segment (start 154.1 151) (end 154.1 151.45) (width 0.2) (layer F.Cu) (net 7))
 (segment (start 154 151.55) (end 153 151.55) (width 0.2) (layer F.Cu) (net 7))
 (segment (start 154.1 151.45) (end 154 151.55) (width 0.2) (layer F.Cu) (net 7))
 (segment (start 152.204199 152.404199) (end 153 151.55) (width 0.2) (layer F.Cu) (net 7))
 (segment (start 147.875 154.335) (end 148.465 154.335) (width 0.2) (layer B.Cu) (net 7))
 (segment (start 148.465 154.335) (end 148.75 154.05) (width 0.2) (layer B.Cu) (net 7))
 (segment (start 148.75 153.45) (end 148.8 153.4) (width 0.2) (layer B.Cu) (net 7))
 (segment (start 148.75 154.05) (end 148.75 153.45) (width 0.2) (layer B.Cu) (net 7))
 (segment (start 148.8 153.4) (end 149.759162 152.450838) (width 0.2) (layer B.Cu) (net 7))
 (via (at 150.68301 153.120839) (size 0.8) (drill 0.4) (layers F.Cu B.Cu) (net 8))
 (segment (start 151.55 152.253849) (end 151.55 151) (width 0.2) (layer F.Cu) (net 8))
 (segment (start 150.68301 153.120839) (end 151.55 152.253849) (width 0.2) (layer F.Cu) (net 8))
 (segment (start 150.579161 153.120839) (end 150.68301 153.120839) (width 0.2) (layer B.Cu) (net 8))
 (segment (start 149.25 154.45) (end 150.579161 153.120839) (width 0.2) (layer B.Cu) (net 8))
 (segment (start 149.25 155.3) (end 149.25 154.45) (width 0.2) (layer B.Cu) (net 8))
 (segment (start 148.945 155.605) (end 149.25 155.3) (width 0.2) (layer B.Cu) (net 8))
 (segment (start 147.875 155.605) (end 148.945 155.605) (width 0.2) (layer B.Cu) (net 8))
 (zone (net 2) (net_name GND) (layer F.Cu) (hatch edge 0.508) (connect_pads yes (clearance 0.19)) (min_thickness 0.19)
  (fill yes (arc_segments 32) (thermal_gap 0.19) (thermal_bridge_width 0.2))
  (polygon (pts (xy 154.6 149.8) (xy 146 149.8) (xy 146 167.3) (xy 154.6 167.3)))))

